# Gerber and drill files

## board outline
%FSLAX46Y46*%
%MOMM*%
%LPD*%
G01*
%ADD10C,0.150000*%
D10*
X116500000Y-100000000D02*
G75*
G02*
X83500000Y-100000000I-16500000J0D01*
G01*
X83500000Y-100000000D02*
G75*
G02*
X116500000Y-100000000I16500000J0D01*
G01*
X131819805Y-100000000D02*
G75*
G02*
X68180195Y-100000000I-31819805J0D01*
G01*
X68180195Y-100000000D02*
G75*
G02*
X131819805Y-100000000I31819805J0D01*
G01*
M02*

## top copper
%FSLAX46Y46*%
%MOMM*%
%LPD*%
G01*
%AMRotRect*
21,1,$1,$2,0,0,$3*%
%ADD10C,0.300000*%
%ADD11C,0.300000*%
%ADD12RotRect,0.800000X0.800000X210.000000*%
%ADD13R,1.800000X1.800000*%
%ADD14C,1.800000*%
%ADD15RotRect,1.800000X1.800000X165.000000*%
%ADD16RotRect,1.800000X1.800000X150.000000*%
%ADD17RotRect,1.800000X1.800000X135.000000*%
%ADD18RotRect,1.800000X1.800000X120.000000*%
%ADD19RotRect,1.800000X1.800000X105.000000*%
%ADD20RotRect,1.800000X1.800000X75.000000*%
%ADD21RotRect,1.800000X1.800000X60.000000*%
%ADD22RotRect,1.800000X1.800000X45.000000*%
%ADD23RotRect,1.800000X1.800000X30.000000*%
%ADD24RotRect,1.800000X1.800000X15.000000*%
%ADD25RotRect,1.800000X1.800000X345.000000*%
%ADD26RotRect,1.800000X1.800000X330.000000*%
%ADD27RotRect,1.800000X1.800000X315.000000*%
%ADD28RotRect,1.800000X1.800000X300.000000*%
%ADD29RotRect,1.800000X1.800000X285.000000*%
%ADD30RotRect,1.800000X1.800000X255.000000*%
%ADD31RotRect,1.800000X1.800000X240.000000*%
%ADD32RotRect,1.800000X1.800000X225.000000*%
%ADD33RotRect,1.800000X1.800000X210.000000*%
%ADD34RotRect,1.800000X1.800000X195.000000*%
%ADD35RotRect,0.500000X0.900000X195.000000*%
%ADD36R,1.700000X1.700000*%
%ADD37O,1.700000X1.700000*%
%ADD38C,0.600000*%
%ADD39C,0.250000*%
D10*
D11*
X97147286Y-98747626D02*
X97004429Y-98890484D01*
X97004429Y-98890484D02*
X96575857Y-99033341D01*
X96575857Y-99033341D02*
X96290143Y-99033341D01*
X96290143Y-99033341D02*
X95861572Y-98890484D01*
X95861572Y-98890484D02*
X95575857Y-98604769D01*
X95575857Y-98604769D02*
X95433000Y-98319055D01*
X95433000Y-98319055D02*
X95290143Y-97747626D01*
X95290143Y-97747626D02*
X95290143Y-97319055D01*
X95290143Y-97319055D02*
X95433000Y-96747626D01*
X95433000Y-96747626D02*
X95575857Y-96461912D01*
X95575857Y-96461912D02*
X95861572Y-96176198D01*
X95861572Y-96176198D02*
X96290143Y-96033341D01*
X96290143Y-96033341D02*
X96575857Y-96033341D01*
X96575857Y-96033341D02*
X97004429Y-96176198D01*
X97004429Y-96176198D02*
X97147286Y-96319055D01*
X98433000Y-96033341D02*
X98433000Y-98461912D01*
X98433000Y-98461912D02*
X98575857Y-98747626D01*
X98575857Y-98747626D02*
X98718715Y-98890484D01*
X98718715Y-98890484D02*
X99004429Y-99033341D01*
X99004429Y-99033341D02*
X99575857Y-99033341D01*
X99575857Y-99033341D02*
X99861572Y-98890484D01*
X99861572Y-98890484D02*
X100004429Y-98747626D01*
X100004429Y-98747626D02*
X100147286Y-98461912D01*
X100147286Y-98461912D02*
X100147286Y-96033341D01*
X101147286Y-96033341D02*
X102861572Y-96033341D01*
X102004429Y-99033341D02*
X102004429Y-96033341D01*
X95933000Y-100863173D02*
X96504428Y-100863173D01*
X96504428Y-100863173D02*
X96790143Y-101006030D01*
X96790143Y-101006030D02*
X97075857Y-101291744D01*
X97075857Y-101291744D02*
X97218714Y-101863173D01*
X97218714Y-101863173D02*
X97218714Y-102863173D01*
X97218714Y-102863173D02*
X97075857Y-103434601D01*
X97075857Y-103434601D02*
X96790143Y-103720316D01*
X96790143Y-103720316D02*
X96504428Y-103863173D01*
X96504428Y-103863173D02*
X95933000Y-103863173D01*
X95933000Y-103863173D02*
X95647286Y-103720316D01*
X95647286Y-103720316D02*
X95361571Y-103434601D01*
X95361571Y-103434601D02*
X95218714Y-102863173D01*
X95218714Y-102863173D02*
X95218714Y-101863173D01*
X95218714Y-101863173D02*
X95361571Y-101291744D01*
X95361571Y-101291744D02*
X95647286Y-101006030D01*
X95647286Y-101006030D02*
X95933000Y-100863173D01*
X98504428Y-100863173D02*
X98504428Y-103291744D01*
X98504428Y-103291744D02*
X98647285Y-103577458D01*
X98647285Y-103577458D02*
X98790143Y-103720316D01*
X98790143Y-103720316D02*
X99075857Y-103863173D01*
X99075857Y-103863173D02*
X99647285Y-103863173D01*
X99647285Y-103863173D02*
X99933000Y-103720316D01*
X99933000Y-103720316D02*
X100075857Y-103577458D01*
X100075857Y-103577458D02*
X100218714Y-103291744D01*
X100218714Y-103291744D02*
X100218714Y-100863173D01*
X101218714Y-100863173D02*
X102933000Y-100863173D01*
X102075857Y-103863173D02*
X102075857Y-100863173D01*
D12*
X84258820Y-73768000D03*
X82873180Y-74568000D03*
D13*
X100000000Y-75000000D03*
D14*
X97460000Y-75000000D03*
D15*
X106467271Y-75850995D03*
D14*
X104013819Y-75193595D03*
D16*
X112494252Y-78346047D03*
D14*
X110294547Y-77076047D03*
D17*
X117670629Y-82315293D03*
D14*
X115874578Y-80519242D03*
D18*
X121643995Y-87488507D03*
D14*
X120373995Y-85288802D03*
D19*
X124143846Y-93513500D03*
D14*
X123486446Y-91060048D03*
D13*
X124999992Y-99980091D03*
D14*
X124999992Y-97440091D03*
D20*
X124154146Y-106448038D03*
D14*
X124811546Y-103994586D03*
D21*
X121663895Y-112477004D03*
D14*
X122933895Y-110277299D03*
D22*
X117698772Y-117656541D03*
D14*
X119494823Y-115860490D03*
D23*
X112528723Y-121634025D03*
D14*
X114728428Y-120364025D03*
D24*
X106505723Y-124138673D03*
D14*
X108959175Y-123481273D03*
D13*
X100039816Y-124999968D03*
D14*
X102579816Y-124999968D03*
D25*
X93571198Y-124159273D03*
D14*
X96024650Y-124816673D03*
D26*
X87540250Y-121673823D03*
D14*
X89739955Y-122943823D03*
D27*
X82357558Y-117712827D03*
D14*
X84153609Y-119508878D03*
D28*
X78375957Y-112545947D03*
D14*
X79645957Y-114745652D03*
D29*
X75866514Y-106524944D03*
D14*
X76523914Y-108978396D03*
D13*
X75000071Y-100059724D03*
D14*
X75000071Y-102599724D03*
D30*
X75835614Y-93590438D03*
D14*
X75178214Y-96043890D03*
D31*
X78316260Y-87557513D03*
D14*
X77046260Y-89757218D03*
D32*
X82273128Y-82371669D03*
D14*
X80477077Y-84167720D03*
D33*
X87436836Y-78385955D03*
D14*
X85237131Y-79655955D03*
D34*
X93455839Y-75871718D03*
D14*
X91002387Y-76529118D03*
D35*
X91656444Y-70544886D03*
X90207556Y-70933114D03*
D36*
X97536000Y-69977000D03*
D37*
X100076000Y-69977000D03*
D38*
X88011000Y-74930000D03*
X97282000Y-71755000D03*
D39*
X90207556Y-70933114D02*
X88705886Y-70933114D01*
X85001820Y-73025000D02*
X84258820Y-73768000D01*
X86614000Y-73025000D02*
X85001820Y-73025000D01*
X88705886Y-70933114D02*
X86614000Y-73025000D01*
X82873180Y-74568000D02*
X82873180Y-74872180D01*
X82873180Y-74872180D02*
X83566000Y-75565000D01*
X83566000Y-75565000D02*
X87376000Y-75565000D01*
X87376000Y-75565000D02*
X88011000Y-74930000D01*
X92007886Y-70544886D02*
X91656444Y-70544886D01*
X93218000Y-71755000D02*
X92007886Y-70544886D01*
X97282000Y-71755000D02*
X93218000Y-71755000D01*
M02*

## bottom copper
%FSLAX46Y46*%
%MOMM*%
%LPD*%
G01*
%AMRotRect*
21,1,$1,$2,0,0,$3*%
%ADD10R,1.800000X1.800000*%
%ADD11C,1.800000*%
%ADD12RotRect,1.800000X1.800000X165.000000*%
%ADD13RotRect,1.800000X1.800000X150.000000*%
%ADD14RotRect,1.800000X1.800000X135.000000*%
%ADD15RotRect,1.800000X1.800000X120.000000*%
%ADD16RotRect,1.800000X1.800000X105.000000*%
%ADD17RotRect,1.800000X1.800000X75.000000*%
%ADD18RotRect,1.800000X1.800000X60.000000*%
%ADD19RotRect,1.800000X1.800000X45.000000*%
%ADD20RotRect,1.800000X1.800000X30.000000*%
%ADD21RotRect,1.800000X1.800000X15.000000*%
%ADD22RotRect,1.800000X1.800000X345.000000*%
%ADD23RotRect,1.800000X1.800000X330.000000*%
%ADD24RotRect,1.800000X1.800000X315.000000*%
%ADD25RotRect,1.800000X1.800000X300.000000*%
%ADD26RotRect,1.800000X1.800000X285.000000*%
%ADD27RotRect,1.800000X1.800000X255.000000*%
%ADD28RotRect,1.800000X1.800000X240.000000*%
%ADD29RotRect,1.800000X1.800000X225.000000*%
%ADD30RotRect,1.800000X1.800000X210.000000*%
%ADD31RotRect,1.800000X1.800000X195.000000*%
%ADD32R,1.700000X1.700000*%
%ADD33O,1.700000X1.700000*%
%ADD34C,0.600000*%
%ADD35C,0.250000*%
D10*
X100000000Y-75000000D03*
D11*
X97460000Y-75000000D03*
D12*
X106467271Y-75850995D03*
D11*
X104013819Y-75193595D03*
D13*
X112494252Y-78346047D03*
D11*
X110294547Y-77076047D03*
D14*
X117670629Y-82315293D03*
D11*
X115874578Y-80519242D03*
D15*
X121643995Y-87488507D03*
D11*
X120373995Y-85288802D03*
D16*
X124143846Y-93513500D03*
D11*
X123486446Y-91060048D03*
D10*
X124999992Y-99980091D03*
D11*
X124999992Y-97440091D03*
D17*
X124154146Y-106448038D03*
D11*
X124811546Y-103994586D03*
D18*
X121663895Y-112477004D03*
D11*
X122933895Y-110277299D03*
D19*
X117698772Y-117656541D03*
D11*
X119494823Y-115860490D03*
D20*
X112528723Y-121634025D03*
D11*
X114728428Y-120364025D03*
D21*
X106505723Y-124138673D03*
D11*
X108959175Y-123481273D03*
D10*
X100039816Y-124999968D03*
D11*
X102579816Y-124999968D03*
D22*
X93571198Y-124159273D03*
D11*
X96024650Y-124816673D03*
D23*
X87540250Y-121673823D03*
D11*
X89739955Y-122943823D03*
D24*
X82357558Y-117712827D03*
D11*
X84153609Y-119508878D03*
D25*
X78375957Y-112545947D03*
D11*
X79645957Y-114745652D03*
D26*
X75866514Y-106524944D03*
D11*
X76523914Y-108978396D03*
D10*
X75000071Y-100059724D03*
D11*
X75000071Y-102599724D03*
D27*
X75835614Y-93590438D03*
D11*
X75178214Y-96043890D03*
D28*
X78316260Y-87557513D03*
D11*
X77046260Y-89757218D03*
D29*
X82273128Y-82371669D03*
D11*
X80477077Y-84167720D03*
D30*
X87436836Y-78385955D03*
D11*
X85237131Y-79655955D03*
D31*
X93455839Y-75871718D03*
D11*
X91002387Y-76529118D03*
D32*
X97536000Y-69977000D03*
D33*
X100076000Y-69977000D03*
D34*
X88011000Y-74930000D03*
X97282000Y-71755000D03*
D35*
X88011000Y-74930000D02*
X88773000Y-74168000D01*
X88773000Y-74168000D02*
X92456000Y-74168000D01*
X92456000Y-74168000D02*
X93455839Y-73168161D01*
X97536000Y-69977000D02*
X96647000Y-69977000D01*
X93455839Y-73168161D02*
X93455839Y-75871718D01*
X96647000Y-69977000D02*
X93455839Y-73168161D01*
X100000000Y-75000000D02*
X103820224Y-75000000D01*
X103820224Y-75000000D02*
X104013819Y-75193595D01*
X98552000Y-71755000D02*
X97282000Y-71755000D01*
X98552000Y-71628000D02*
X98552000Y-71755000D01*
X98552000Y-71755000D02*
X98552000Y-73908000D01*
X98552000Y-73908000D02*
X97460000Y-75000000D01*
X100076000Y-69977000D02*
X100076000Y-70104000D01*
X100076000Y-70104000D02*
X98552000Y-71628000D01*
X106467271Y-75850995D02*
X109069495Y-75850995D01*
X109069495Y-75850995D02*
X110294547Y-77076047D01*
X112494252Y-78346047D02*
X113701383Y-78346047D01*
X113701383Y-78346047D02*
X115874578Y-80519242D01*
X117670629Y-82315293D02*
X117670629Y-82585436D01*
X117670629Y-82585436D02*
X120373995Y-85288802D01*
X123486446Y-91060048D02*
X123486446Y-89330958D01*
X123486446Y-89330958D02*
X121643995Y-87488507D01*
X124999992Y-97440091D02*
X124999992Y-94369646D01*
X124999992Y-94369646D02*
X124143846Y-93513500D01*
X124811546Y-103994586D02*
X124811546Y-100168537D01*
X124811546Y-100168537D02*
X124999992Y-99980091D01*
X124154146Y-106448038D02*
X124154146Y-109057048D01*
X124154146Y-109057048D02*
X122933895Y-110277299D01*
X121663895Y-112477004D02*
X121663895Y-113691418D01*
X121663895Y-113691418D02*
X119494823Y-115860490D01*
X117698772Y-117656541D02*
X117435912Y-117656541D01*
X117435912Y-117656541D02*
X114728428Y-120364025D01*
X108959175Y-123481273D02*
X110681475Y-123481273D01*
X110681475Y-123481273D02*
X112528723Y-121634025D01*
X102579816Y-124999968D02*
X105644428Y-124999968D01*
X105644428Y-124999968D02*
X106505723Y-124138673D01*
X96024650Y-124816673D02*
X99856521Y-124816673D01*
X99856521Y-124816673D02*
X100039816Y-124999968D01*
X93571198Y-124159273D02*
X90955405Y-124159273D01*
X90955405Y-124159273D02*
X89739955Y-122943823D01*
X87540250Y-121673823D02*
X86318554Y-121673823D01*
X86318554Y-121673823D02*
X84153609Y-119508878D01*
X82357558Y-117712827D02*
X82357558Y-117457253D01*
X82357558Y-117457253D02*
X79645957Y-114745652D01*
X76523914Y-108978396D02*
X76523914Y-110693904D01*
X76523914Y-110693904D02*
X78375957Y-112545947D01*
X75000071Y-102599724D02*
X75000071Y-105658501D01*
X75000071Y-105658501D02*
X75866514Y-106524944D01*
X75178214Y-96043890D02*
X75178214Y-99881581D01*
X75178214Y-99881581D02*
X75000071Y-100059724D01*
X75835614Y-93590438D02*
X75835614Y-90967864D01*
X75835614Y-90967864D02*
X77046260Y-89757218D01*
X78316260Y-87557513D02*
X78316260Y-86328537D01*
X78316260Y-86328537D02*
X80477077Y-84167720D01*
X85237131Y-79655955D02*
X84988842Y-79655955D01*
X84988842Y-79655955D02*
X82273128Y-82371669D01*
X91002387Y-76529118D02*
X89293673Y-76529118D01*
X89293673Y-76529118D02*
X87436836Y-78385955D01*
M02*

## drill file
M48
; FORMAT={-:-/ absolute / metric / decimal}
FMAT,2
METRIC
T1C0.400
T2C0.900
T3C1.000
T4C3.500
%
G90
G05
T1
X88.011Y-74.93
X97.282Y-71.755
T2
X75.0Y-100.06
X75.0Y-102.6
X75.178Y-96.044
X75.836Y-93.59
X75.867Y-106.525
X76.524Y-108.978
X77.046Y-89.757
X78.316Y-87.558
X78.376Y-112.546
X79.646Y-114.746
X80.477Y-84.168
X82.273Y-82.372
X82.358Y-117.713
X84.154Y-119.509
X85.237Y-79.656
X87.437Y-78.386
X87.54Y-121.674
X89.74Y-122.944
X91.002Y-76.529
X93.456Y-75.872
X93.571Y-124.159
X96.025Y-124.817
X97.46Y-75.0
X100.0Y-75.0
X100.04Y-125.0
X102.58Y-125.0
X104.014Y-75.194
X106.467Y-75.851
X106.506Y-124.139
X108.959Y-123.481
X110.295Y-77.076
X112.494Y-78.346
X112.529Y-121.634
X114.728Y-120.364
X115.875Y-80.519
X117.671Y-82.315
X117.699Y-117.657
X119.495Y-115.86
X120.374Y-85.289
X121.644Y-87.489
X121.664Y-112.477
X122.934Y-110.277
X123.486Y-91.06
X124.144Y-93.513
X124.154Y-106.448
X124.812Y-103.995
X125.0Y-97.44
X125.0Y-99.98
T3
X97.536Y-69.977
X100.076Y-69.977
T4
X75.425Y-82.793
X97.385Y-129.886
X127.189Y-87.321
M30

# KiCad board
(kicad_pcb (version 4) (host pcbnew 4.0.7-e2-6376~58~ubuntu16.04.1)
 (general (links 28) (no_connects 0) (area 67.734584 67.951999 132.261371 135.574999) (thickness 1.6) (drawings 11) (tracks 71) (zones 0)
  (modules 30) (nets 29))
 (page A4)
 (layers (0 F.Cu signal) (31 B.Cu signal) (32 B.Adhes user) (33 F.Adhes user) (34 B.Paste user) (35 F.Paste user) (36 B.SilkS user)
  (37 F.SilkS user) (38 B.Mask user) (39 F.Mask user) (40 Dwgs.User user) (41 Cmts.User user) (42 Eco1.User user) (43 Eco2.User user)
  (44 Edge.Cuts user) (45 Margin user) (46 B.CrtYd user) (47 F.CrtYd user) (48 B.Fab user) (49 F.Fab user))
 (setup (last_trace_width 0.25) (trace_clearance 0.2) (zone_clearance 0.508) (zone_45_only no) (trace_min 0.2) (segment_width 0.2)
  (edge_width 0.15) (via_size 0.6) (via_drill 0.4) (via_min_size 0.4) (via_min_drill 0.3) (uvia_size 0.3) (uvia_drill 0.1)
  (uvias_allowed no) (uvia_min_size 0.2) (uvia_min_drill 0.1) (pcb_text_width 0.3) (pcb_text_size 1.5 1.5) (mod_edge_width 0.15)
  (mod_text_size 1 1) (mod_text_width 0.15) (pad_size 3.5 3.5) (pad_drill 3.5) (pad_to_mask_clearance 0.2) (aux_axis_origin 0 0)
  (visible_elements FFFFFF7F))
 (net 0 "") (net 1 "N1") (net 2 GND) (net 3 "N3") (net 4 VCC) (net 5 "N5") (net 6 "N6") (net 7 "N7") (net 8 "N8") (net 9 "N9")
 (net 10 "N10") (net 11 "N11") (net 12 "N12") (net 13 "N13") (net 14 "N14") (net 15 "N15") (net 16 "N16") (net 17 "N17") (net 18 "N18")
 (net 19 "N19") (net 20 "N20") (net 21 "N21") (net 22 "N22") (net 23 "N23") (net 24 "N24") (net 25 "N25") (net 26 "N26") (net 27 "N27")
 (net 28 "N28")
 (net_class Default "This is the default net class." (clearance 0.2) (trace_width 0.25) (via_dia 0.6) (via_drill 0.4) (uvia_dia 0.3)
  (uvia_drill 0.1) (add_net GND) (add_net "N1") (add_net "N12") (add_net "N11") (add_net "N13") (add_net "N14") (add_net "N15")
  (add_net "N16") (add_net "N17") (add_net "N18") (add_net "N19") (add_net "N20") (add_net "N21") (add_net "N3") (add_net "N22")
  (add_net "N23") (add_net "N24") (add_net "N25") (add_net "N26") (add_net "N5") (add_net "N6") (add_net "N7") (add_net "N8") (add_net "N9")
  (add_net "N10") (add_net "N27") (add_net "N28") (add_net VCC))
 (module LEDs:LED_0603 (layer F.Cu) (at 83.566 74.168 30)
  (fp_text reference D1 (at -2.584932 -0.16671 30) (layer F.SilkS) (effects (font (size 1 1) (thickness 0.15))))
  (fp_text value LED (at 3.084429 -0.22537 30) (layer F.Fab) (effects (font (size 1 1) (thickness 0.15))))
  (pad 2 smd rect (at 0.8 0 210) (size 0.8 0.8) (layers F.Cu F.Paste F.Mask) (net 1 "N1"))
  (pad 1 smd rect (at -0.8 0 210) (size 0.8 0.8) (layers F.Cu F.Paste F.Mask) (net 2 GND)))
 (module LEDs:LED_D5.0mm (layer F.Cu) (at 100 75 180)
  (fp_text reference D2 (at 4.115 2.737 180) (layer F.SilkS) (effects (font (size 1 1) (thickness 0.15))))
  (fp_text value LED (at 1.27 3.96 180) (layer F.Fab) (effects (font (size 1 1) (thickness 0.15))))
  (pad 1 thru_hole rect (at 0 0 180) (size 1.8 1.8) (drill 0.9) (layers *.Cu *.Mask) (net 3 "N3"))
  (pad 2 thru_hole circle (at 2.54 0 180) (size 1.8 1.8) (drill 0.9) (layers *.Cu *.Mask) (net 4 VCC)))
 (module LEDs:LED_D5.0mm (layer F.Cu) (at 106.467271 75.850995 165)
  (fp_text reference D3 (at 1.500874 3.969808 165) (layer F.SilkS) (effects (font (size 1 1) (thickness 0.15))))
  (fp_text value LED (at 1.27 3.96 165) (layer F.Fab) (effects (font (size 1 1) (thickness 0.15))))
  (pad 1 thru_hole rect (at 0 0 165) (size 1.8 1.8) (drill 0.9) (layers *.Cu *.Mask) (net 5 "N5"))
  (pad 2 thru_hole circle (at 2.54 0 165) (size 1.8 1.8) (drill 0.9) (layers *.Cu *.Mask) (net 3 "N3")))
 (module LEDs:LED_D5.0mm (layer F.Cu) (at 112.494252 78.346047 150)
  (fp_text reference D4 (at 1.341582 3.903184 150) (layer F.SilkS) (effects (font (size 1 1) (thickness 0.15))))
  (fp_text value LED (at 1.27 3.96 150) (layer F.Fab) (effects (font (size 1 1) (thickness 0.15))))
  (pad 1 thru_hole rect (at 0 0 150) (size 1.8 1.8) (drill 0.9) (layers *.Cu *.Mask) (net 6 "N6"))
  (pad 2 thru_hole circle (at 2.54 0 150) (size 1.8 1.8) (drill 0.9) (layers *.Cu *.Mask) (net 5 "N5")))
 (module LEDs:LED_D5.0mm (layer F.Cu) (at 117.670629 82.315293 135)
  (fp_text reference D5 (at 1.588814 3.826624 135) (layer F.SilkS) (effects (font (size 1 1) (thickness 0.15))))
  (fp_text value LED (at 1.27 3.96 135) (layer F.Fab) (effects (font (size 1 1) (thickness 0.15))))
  (pad 1 thru_hole rect (at 0 0 135) (size 1.8 1.8) (drill 0.9) (layers *.Cu *.Mask) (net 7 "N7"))
  (pad 2 thru_hole circle (at 2.54 0 135) (size 1.8 1.8) (drill 0.9) (layers *.Cu *.Mask) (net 6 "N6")))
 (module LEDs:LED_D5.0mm (layer F.Cu) (at 121.643995 87.488507 120)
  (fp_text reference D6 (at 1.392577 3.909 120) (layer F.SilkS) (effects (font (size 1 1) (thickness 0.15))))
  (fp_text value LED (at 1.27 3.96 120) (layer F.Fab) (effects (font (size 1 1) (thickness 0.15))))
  (pad 1 thru_hole rect (at 0 0 120) (size 1.8 1.8) (drill 0.9) (layers *.Cu *.Mask) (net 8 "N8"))
  (pad 2 thru_hole circle (at 2.54 0 120) (size 1.8 1.8) (drill 0.9) (layers *.Cu *.Mask) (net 7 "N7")))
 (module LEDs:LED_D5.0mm (layer F.Cu) (at 124.143846 93.5135 105)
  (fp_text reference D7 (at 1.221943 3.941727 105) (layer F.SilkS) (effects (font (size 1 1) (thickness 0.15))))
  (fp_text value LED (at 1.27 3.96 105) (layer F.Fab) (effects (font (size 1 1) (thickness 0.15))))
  (pad 1 thru_hole rect (at 0 0 105) (size 1.8 1.8) (drill 0.9) (layers *.Cu *.Mask) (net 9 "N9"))
  (pad 2 thru_hole circle (at 2.54 0 105) (size 1.8 1.8) (drill 0.9) (layers *.Cu *.Mask) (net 8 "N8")))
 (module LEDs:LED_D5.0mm (layer F.Cu) (at 124.999992 99.980091 90)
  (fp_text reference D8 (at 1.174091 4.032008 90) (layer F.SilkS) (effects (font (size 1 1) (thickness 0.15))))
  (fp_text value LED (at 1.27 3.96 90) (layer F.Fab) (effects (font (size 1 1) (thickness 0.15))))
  (pad 1 thru_hole rect (at 0 0 90) (size 1.8 1.8) (drill 0.9) (layers *.Cu *.Mask) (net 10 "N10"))
  (pad 2 thru_hole circle (at 2.54 0 90) (size 1.8 1.8) (drill 0.9) (layers *.Cu *.Mask) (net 9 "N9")))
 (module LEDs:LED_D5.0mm (layer F.Cu) (at 124.154146 106.448038 75)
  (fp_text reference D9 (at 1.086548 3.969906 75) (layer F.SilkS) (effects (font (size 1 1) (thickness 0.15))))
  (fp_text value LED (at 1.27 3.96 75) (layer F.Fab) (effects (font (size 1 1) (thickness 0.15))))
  (pad 1 thru_hole rect (at 0 0 75) (size 1.8 1.8) (drill 0.9) (layers *.Cu *.Mask) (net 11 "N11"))
  (pad 2 thru_hole circle (at 2.54 0 75) (size 1.8 1.8) (drill 0.9) (layers *.Cu *.Mask) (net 10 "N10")))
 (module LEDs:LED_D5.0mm (layer F.Cu) (at 121.663895 112.477004 60)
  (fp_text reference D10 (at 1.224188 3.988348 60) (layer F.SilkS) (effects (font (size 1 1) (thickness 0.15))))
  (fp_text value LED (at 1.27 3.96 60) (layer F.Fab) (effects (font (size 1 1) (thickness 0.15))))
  (pad 1 thru_hole rect (at 0 0 60) (size 1.8 1.8) (drill 0.9) (layers *.Cu *.Mask) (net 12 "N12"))
  (pad 2 thru_hole circle (at 2.54 0 60) (size 1.8 1.8) (drill 0.9) (layers *.Cu *.Mask) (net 11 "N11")))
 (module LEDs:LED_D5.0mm (layer F.Cu) (at 117.698772 117.656541 45)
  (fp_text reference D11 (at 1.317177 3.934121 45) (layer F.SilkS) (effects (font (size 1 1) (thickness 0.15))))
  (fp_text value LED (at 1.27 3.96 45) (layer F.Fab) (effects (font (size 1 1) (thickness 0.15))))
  (pad 1 thru_hole rect (at 0 0 45) (size 1.8 1.8) (drill 0.9) (layers *.Cu *.Mask) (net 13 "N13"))
  (pad 2 thru_hole circle (at 2.54 0 45) (size 1.8 1.8) (drill 0.9) (layers *.Cu *.Mask) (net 12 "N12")))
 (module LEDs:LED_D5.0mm (layer F.Cu) (at 112.528723 121.634025 30)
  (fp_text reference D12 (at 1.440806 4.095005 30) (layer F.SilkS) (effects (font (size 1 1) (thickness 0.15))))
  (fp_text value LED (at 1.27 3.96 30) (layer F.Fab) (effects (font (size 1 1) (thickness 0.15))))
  (pad 1 thru_hole rect (at 0 0 30) (size 1.8 1.8) (drill 0.9) (layers *.Cu *.Mask) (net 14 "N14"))
  (pad 2 thru_hole circle (at 2.54 0 30) (size 1.8 1.8) (drill 0.9) (layers *.Cu *.Mask) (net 13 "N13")))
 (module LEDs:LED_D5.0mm (layer F.Cu) (at 106.505723 124.138673 15)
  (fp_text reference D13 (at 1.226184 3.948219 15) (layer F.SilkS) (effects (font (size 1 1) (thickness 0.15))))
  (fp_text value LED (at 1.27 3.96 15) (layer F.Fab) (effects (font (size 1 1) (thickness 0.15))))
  (pad 1 thru_hole rect (at 0 0 15) (size 1.8 1.8) (drill 0.9) (layers *.Cu *.Mask) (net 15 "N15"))
  (pad 2 thru_hole circle (at 2.54 0 15) (size 1.8 1.8) (drill 0.9) (layers *.Cu *.Mask) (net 14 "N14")))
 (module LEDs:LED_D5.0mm (layer F.Cu) (at 100.039816 124.999968)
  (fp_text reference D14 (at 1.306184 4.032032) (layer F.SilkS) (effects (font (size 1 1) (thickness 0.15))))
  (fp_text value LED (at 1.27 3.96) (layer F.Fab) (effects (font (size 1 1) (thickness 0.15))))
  (pad 1 thru_hole rect (at 0 0) (size 1.8 1.8) (drill 0.9) (layers *.Cu *.Mask) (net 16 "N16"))
  (pad 2 thru_hole circle (at 2.54 0) (size 1.8 1.8) (drill 0.9) (layers *.Cu *.Mask) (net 15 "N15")))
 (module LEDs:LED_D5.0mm (layer F.Cu) (at 93.571198 124.159273 345)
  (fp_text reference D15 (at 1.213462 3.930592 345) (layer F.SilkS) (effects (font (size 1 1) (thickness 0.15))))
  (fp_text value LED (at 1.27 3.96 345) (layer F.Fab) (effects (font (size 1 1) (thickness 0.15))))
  (pad 1 thru_hole rect (at 0 0 345) (size 1.8 1.8) (drill 0.9) (layers *.Cu *.Mask) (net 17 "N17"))
  (pad 2 thru_hole circle (at 2.54 0 345) (size 1.8 1.8) (drill 0.9) (layers *.Cu *.Mask) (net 16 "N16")))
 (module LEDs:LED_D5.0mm (layer F.Cu) (at 87.54025 121.673823 330)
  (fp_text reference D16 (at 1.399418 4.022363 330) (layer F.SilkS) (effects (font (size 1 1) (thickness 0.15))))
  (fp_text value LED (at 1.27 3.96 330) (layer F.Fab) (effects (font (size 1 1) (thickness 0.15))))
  (pad 1 thru_hole rect (at 0 0 330) (size 1.8 1.8) (drill 0.9) (layers *.Cu *.Mask) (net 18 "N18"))
  (pad 2 thru_hole circle (at 2.54 0 330) (size 1.8 1.8) (drill 0.9) (layers *.Cu *.Mask) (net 17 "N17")))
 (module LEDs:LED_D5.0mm (layer F.Cu) (at 82.357558 117.712827 315)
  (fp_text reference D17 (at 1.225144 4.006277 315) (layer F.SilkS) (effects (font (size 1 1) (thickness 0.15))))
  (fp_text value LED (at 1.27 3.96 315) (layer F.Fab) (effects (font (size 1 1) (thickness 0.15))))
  (pad 1 thru_hole rect (at 0 0 315) (size 1.8 1.8) (drill 0.9) (layers *.Cu *.Mask) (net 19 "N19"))
  (pad 2 thru_hole circle (at 2.54 0 315) (size 1.8 1.8) (drill 0.9) (layers *.Cu *.Mask) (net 18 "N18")))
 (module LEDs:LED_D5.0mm (layer F.Cu) (at 78.375957 112.545947 300)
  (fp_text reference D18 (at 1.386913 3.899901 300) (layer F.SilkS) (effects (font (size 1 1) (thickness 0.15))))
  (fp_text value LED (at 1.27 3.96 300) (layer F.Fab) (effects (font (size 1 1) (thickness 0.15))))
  (pad 1 thru_hole rect (at 0 0 300) (size 1.8 1.8) (drill 0.9) (layers *.Cu *.Mask) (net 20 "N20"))
  (pad 2 thru_hole circle (at 2.54 0 300) (size 1.8 1.8) (drill 0.9) (layers *.Cu *.Mask) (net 19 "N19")))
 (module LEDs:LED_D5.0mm (layer F.Cu) (at 75.866514 106.524944 285)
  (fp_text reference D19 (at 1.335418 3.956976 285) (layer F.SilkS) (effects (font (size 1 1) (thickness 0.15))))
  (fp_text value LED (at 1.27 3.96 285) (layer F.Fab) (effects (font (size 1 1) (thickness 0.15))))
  (pad 1 thru_hole rect (at 0 0 285) (size 1.8 1.8) (drill 0.9) (layers *.Cu *.Mask) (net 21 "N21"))
  (pad 2 thru_hole circle (at 2.54 0 285) (size 1.8 1.8) (drill 0.9) (layers *.Cu *.Mask) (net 20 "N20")))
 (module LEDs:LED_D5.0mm (layer F.Cu) (at 75.000071 100.059724 270)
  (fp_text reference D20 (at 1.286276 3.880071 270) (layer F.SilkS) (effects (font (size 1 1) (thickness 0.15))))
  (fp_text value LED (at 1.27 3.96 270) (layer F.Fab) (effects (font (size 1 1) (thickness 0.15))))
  (pad 1 thru_hole rect (at 0 0 270) (size 1.8 1.8) (drill 0.9) (layers *.Cu *.Mask) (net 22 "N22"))
  (pad 2 thru_hole circle (at 2.54 0 270) (size 1.8 1.8) (drill 0.9) (layers *.Cu *.Mask) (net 21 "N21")))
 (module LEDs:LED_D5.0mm (layer F.Cu) (at 75.835614 93.590438 255)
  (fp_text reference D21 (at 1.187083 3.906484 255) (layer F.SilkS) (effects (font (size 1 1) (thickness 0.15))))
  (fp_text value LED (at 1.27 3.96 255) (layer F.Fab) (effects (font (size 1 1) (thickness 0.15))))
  (pad 1 thru_hole rect (at 0 0 255) (size 1.8 1.8) (drill 0.9) (layers *.Cu *.Mask) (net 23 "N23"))
  (pad 2 thru_hole circle (at 2.54 0 255) (size 1.8 1.8) (drill 0.9) (layers *.Cu *.Mask) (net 22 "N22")))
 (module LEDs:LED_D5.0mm (layer F.Cu) (at 78.31626 87.557513 240)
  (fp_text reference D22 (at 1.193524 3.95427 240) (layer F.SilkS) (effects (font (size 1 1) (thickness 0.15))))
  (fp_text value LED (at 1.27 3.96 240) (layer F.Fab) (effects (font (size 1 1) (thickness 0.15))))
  (pad 1 thru_hole rect (at 0 0 240) (size 1.8 1.8) (drill 0.9) (layers *.Cu *.Mask) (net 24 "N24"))
  (pad 2 thru_hole circle (at 2.54 0 240) (size 1.8 1.8) (drill 0.9) (layers *.Cu *.Mask) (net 23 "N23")))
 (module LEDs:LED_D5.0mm (layer F.Cu) (at 82.273128 82.371669 225)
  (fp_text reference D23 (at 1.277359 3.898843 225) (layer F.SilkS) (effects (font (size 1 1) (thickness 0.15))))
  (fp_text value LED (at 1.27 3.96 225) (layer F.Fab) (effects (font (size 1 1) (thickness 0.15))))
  (pad 1 thru_hole rect (at 0 0 225) (size 1.8 1.8) (drill 0.9) (layers *.Cu *.Mask) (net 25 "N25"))
  (pad 2 thru_hole circle (at 2.54 0 225) (size 1.8 1.8) (drill 0.9) (layers *.Cu *.Mask) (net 24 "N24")))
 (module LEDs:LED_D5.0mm (layer F.Cu) (at 87.436836 78.385955 210)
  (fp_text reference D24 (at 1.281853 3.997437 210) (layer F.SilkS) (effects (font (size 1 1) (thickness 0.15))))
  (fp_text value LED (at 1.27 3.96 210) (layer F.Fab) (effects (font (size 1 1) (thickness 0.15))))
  (pad 1 thru_hole rect (at 0 0 210) (size 1.8 1.8) (drill 0.9) (layers *.Cu *.Mask) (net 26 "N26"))
  (pad 2 thru_hole circle (at 2.54 0 210) (size 1.8 1.8) (drill 0.9) (layers *.Cu *.Mask) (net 25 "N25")))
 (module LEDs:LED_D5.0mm (layer F.Cu) (at 93.455839 75.871718 195)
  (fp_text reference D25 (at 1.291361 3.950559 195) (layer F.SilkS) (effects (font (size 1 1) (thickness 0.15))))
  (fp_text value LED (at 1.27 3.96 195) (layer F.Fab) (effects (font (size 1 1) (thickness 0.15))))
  (pad 1 thru_hole rect (at 0 0 195) (size 1.8 1.8) (drill 0.9) (layers *.Cu *.Mask) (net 2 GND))
  (pad 2 thru_hole circle (at 2.54 0 195) (size 1.8 1.8) (drill 0.9) (layers *.Cu *.Mask) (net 26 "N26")))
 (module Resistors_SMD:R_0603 (layer F.Cu) (at 90.932 70.739 195)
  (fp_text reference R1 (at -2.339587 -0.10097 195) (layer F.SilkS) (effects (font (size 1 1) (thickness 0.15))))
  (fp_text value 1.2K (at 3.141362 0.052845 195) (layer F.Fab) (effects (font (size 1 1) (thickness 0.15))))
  (pad 1 smd rect (at -0.75 0 195) (size 0.5 0.9) (layers F.Cu F.Paste F.Mask) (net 4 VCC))
  (pad 2 smd rect (at 0.75 0 195) (size 0.5 0.9) (layers F.Cu F.Paste F.Mask) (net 1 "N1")))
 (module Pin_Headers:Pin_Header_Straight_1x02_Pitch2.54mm (layer F.Cu) (at 97.536 69.977 90)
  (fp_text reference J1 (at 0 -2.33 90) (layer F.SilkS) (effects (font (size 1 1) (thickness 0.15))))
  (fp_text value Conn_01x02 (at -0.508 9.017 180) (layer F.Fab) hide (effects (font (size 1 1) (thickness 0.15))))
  (pad 1 thru_hole rect (at 0 0 90) (size 1.7 1.7) (drill 1) (layers *.Cu *.Mask) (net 2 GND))
  (pad 2 thru_hole oval (at 0 2.54 90) (size 1.7 1.7) (drill 1) (layers *.Cu *.Mask) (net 4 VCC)))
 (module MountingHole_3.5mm (layer F.Cu) (at 97.385327 129.88584)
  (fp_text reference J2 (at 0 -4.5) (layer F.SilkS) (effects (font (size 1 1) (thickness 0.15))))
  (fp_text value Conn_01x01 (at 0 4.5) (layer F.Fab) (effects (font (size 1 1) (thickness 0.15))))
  (pad 1 np_thru_hole circle (at 0 0) (size 3.5 3.5) (drill 3.5) (layers *.Cu *.Mask) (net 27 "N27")))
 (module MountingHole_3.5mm (layer F.Cu) (at 127.189233 87.321452)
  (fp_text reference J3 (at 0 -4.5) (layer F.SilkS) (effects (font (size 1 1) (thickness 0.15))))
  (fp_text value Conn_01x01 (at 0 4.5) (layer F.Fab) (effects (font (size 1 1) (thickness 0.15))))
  (pad "" np_thru_hole circle (at 0 0) (size 3.5 3.5) (drill 3.5) (layers *.Cu *.Mask)))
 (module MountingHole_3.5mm (layer F.Cu) (at 75.425438 82.792706)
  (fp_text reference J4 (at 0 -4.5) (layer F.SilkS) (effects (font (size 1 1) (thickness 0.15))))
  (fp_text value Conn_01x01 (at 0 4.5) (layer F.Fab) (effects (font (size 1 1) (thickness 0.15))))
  (pad 1 np_thru_hole circle (at 0 0) (size 3.5 3.5) (drill 3.5) (layers *.Cu *.Mask) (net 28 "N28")))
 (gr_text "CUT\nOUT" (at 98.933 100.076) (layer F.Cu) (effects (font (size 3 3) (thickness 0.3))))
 (gr_circle (center 100 100) (end 116.5 100) (layer Edge.Cuts) (width 0.15))
 (gr_circle (center 100 100) (end 122.5 122.5) (layer Edge.Cuts) (width 0.15))
 (segment (start 90.207556 70.933114) (end 88.705886 70.933114) (width 0.25) (layer F.Cu) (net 1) (status 10))
 (segment (start 85.00182 73.025) (end 84.25882 73.768) (width 0.25) (layer F.Cu) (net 1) (status 20))
 (segment (start 86.614 73.025) (end 85.00182 73.025) (width 0.25) (layer F.Cu) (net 1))
 (segment (start 88.705886 70.933114) (end 86.614 73.025) (width 0.25) (layer F.Cu) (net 1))
 (segment (start 82.87318 74.568) (end 82.87318 74.87218) (width 0.25) (layer F.Cu) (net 2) (status 30))
 (segment (start 82.87318 74.87218) (end 83.566 75.565) (width 0.25) (layer F.Cu) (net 2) (status 10))
 (segment (start 83.566 75.565) (end 87.376 75.565) (width 0.25) (layer F.Cu) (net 2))
 (segment (start 87.376 75.565) (end 88.011 74.93) (width 0.25) (layer F.Cu) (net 2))
 (via (at 88.011 74.93) (size 0.6) (drill 0.4) (layers F.Cu B.Cu) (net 2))
 (segment (start 88.011 74.93) (end 88.773 74.168) (width 0.25) (layer B.Cu) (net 2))
 (segment (start 88.773 74.168) (end 92.456 74.168) (width 0.25) (layer B.Cu) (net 2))
 (segment (start 92.456 74.168) (end 93.455839 73.168161) (width 0.25) (layer B.Cu) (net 2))
 (segment (start 97.536 69.977) (end 96.647 69.977) (width 0.25) (layer B.Cu) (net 2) (status 10))
 (segment (start 93.455839 73.168161) (end 93.455839 75.871718) (width 0.25) (layer B.Cu) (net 2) (status 20))
 (segment (start 96.647 69.977) (end 93.455839 73.168161) (width 0.25) (layer B.Cu) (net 2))
 (segment (start 100 75) (end 103.820224 75) (width 0.25) (layer B.Cu) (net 3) (status 30))
 (segment (start 103.820224 75) (end 104.013819 75.193595) (width 0.25) (layer B.Cu) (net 3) (status 30))
 (segment (start 98.552 71.755) (end 97.282 71.755) (width 0.25) (layer B.Cu) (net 4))
 (segment (start 92.007886 70.544886) (end 91.656444 70.544886) (width 0.25) (layer F.Cu) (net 4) (status 20))
 (segment (start 93.218 71.755) (end 92.007886 70.544886) (width 0.25) (layer F.Cu) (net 4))
 (segment (start 97.282 71.755) (end 93.218 71.755) (width 0.25) (layer F.Cu) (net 4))
 (via (at 97.282 71.755) (size 0.6) (drill 0.4) (layers F.Cu B.Cu) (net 4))
 (segment (start 98.552 71.628) (end 98.552 71.755) (width 0.25) (layer B.Cu) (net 4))
 (segment (start 98.552 71.755) (end 98.552 73.908) (width 0.25) (layer B.Cu) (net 4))
 (segment (start 98.552 73.908) (end 97.46 75) (width 0.25) (layer B.Cu) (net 4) (status 20))
 (segment (start 100.076 69.977) (end 100.076 70.104) (width 0.25) (layer B.Cu) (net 4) (status 30))
 (segment (start 100.076 70.104) (end 98.552 71.628) (width 0.25) (layer B.Cu) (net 4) (status 10))
 (segment (start 106.467271 75.850995) (end 109.069495 75.850995) (width 0.25) (layer B.Cu) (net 5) (status 10))
 (segment (start 109.069495 75.850995) (end 110.294547 77.076047) (width 0.25) (layer B.Cu) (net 5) (status 20))
 (segment (start 112.494252 78.346047) (end 113.701383 78.346047) (width 0.25) (layer B.Cu) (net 6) (status 10))
 (segment (start 113.701383 78.346047) (end 115.874578 80.519242) (width 0.25) (layer B.Cu) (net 6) (status 20))
 (segment (start 117.670629 82.315293) (end 117.670629 82.585436) (width 0.25) (layer B.Cu) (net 7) (status 30))
 (segment (start 117.670629 82.585436) (end 120.373995 85.288802) (width 0.25) (layer B.Cu) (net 7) (status 30))
 (segment (start 123.486446 91.060048) (end 123.486446 89.330958) (width 0.25) (layer B.Cu) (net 8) (status 10))
 (segment (start 123.486446 89.330958) (end 121.643995 87.488507) (width 0.25) (layer B.Cu) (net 8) (status 20))
 (segment (start 124.999992 97.440091) (end 124.999992 94.369646) (width 0.25) (layer B.Cu) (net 9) (status 10))
 (segment (start 124.999992 94.369646) (end 124.143846 93.5135) (width 0.25) (layer B.Cu) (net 9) (status 20))
 (segment (start 124.811546 103.994586) (end 124.811546 100.168537) (width 0.25) (layer B.Cu) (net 10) (status 30))
 (segment (start 124.811546 100.168537) (end 124.999992 99.980091) (width 0.25) (layer B.Cu) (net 10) (status 30))
 (segment (start 124.154146 106.448038) (end 124.154146 109.057048) (width 0.25) (layer B.Cu) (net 11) (status 10))
 (segment (start 124.154146 109.057048) (end 122.933895 110.277299) (width 0.25) (layer B.Cu) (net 11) (status 20))
 (segment (start 121.663895 112.477004) (end 121.663895 113.691418) (width 0.25) (layer B.Cu) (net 12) (status 10))
 (segment (start 121.663895 113.691418) (end 119.494823 115.86049) (width 0.25) (layer B.Cu) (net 12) (status 20))
 (segment (start 117.698772 117.656541) (end 117.435912 117.656541) (width 0.25) (layer B.Cu) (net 13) (status 30))
 (segment (start 117.435912 117.656541) (end 114.728428 120.364025) (width 0.25) (layer B.Cu) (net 13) (status 30))
 (segment (start 108.959175 123.481273) (end 110.681475 123.481273) (width 0.25) (layer B.Cu) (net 14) (status 10))
 (segment (start 110.681475 123.481273) (end 112.528723 121.634025) (width 0.25) (layer B.Cu) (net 14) (status 20))
 (segment (start 102.579816 124.999968) (end 105.644428 124.999968) (width 0.25) (layer B.Cu) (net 15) (status 10))
 (segment (start 105.644428 124.999968) (end 106.505723 124.138673) (width 0.25) (layer B.Cu) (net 15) (status 20))
 (segment (start 96.02465 124.816673) (end 99.856521 124.816673) (width 0.25) (layer B.Cu) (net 16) (status 30))
 (segment (start 99.856521 124.816673) (end 100.039816 124.999968) (width 0.25) (layer B.Cu) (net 16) (status 30))
 (segment (start 93.571198 124.159273) (end 90.955405 124.159273) (width 0.25) (layer B.Cu) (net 17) (status 10))
 (segment (start 90.955405 124.159273) (end 89.739955 122.943823) (width 0.25) (layer B.Cu) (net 17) (status 20))
 (segment (start 87.54025 121.673823) (end 86.318554 121.673823) (width 0.25) (layer B.Cu) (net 18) (status 10))
 (segment (start 86.318554 121.673823) (end 84.153609 119.508878) (width 0.25) (layer B.Cu) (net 18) (status 20))
 (segment (start 82.357558 117.712827) (end 82.357558 117.457253) (width 0.25) (layer B.Cu) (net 19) (status 30))
 (segment (start 82.357558 117.457253) (end 79.645957 114.745652) (width 0.25) (layer B.Cu) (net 19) (status 30))
 (segment (start 76.523914 108.978396) (end 76.523914 110.693904) (width 0.25) (layer B.Cu) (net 20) (status 10))
 (segment (start 76.523914 110.693904) (end 78.375957 112.545947) (width 0.25) (layer B.Cu) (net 20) (status 20))
 (segment (start 75.000071 102.599724) (end 75.000071 105.658501) (width 0.25) (layer B.Cu) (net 21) (status 10))
 (segment (start 75.000071 105.658501) (end 75.866514 106.524944) (width 0.25) (layer B.Cu) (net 21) (status 20))
 (segment (start 75.178214 96.04389) (end 75.178214 99.881581) (width 0.25) (layer B.Cu) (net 22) (status 30))
 (segment (start 75.178214 99.881581) (end 75.000071 100.059724) (width 0.25) (layer B.Cu) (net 22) (status 30))
 (segment (start 75.835614 93.590438) (end 75.835614 90.967864) (width 0.25) (layer B.Cu) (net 23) (status 10))
 (segment (start 75.835614 90.967864) (end 77.04626 89.757218) (width 0.25) (layer B.Cu) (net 23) (status 20))
 (segment (start 78.31626 87.557513) (end 78.31626 86.328537) (width 0.25) (layer B.Cu) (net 24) (status 10))
 (segment (start 78.31626 86.328537) (end 80.477077 84.16772) (width 0.25) (layer B.Cu) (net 24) (status 20))
 (segment (start 85.237131 79.655955) (end 84.988842 79.655955) (width 0.25) (layer B.Cu) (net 25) (status 30))
 (segment (start 84.988842 79.655955) (end 82.273128 82.371669) (width 0.25) (layer B.Cu) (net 25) (status 30))
 (segment (start 91.002387 76.529118) (end 89.293673 76.529118) (width 0.25) (layer B.Cu) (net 26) (status 10))
 (segment (start 89.293673 76.529118) (end 87.436836 78.385955) (width 0.25) (layer B.Cu) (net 26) (status 20)))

